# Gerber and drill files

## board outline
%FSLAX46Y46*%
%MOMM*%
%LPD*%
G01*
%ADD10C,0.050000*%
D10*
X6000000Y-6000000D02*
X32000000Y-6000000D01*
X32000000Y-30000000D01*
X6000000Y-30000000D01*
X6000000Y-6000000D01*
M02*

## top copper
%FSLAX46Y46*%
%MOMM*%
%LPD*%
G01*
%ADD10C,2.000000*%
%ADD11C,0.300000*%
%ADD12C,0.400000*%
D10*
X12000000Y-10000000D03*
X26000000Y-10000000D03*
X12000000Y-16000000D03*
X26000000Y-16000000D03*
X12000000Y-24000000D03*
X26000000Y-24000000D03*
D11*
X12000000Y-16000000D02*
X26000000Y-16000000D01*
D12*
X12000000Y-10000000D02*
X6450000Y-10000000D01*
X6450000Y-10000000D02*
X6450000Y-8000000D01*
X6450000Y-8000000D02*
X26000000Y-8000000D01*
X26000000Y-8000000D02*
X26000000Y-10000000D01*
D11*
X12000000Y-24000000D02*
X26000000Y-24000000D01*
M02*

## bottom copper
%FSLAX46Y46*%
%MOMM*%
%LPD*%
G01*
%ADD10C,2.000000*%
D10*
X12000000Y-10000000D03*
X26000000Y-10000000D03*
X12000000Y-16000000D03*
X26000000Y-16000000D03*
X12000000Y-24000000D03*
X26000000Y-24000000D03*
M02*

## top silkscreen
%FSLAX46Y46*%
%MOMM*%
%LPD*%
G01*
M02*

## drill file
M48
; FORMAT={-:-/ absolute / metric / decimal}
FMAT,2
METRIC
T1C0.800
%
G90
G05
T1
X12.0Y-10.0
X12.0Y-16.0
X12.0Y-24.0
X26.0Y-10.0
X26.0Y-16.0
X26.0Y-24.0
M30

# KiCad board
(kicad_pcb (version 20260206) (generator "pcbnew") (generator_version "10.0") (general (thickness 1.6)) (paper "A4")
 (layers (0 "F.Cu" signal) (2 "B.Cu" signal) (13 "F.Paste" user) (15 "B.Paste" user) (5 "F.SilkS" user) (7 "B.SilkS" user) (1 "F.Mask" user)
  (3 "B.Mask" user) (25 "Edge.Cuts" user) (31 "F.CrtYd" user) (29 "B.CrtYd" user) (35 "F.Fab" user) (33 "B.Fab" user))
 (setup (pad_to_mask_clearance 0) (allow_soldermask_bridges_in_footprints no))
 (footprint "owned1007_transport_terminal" (layer "F.Cu") (at 12 10)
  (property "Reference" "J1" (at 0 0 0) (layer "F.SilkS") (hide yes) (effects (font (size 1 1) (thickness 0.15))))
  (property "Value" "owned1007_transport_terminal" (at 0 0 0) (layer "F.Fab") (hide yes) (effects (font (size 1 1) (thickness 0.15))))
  (pad "1" thru_hole circle (at 0 0) (size 2 2) (drill 0.8) (layers "*.Cu" "*.Mask") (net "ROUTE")))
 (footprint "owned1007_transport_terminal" (layer "F.Cu") (at 26 10)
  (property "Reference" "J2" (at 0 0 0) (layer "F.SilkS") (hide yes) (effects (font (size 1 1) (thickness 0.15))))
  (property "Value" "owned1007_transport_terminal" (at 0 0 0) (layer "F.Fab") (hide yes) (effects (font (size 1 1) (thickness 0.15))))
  (pad "1" thru_hole circle (at 0 0) (size 2 2) (drill 0.8) (layers "*.Cu" "*.Mask") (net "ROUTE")))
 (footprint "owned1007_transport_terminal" (layer "F.Cu") (at 12 16)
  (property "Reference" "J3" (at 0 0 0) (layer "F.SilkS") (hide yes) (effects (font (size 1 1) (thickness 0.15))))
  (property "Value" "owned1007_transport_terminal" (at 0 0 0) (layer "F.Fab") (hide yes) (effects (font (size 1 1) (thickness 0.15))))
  (pad "1" thru_hole circle (at 0 0) (size 2 2) (drill 0.8) (layers "*.Cu" "*.Mask") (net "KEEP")))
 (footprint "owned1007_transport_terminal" (layer "F.Cu") (at 26 16)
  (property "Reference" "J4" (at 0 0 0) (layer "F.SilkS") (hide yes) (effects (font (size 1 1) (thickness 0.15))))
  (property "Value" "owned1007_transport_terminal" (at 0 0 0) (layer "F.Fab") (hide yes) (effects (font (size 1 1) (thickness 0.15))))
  (pad "1" thru_hole circle (at 0 0) (size 2 2) (drill 0.8) (layers "*.Cu" "*.Mask") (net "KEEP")))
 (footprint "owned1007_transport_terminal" (layer "F.Cu") (at 12 24)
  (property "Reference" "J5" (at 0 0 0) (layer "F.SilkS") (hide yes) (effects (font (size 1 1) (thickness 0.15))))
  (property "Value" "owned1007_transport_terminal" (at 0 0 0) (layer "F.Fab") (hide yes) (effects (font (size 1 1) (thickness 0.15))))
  (pad "1" thru_hole circle (at 0 0) (size 2 2) (drill 0.8) (layers "*.Cu" "*.Mask") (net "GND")))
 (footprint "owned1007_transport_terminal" (layer "F.Cu") (at 26 24)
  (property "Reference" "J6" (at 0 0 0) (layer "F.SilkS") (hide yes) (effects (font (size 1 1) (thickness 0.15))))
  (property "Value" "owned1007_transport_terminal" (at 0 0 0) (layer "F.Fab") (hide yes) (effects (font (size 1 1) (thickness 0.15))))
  (pad "1" thru_hole circle (at 0 0) (size 2 2) (drill 0.8) (layers "*.Cu" "*.Mask") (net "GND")))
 (gr_rect (start 6 6) (end 32 30) (stroke (width 0.05) (type default)) (fill none) (layer "Edge.Cuts"))
 (segment (start 12 16) (end 26 16) (width 0.3) (layer "F.Cu") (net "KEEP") (locked yes))
 (segment (start 12 10) (end 6.45 10) (width 0.4) (layer "F.Cu") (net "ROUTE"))
 (segment (start 6.45 10) (end 6.45 8) (width 0.4) (layer "F.Cu") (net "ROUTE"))
 (segment (start 6.45 8) (end 26 8) (width 0.4) (layer "F.Cu") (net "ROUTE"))
 (segment (start 26 8) (end 26 10) (width 0.4) (layer "F.Cu") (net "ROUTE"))
 (segment (start 12 24) (end 26 24) (width 0.3) (layer "F.Cu") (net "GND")))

